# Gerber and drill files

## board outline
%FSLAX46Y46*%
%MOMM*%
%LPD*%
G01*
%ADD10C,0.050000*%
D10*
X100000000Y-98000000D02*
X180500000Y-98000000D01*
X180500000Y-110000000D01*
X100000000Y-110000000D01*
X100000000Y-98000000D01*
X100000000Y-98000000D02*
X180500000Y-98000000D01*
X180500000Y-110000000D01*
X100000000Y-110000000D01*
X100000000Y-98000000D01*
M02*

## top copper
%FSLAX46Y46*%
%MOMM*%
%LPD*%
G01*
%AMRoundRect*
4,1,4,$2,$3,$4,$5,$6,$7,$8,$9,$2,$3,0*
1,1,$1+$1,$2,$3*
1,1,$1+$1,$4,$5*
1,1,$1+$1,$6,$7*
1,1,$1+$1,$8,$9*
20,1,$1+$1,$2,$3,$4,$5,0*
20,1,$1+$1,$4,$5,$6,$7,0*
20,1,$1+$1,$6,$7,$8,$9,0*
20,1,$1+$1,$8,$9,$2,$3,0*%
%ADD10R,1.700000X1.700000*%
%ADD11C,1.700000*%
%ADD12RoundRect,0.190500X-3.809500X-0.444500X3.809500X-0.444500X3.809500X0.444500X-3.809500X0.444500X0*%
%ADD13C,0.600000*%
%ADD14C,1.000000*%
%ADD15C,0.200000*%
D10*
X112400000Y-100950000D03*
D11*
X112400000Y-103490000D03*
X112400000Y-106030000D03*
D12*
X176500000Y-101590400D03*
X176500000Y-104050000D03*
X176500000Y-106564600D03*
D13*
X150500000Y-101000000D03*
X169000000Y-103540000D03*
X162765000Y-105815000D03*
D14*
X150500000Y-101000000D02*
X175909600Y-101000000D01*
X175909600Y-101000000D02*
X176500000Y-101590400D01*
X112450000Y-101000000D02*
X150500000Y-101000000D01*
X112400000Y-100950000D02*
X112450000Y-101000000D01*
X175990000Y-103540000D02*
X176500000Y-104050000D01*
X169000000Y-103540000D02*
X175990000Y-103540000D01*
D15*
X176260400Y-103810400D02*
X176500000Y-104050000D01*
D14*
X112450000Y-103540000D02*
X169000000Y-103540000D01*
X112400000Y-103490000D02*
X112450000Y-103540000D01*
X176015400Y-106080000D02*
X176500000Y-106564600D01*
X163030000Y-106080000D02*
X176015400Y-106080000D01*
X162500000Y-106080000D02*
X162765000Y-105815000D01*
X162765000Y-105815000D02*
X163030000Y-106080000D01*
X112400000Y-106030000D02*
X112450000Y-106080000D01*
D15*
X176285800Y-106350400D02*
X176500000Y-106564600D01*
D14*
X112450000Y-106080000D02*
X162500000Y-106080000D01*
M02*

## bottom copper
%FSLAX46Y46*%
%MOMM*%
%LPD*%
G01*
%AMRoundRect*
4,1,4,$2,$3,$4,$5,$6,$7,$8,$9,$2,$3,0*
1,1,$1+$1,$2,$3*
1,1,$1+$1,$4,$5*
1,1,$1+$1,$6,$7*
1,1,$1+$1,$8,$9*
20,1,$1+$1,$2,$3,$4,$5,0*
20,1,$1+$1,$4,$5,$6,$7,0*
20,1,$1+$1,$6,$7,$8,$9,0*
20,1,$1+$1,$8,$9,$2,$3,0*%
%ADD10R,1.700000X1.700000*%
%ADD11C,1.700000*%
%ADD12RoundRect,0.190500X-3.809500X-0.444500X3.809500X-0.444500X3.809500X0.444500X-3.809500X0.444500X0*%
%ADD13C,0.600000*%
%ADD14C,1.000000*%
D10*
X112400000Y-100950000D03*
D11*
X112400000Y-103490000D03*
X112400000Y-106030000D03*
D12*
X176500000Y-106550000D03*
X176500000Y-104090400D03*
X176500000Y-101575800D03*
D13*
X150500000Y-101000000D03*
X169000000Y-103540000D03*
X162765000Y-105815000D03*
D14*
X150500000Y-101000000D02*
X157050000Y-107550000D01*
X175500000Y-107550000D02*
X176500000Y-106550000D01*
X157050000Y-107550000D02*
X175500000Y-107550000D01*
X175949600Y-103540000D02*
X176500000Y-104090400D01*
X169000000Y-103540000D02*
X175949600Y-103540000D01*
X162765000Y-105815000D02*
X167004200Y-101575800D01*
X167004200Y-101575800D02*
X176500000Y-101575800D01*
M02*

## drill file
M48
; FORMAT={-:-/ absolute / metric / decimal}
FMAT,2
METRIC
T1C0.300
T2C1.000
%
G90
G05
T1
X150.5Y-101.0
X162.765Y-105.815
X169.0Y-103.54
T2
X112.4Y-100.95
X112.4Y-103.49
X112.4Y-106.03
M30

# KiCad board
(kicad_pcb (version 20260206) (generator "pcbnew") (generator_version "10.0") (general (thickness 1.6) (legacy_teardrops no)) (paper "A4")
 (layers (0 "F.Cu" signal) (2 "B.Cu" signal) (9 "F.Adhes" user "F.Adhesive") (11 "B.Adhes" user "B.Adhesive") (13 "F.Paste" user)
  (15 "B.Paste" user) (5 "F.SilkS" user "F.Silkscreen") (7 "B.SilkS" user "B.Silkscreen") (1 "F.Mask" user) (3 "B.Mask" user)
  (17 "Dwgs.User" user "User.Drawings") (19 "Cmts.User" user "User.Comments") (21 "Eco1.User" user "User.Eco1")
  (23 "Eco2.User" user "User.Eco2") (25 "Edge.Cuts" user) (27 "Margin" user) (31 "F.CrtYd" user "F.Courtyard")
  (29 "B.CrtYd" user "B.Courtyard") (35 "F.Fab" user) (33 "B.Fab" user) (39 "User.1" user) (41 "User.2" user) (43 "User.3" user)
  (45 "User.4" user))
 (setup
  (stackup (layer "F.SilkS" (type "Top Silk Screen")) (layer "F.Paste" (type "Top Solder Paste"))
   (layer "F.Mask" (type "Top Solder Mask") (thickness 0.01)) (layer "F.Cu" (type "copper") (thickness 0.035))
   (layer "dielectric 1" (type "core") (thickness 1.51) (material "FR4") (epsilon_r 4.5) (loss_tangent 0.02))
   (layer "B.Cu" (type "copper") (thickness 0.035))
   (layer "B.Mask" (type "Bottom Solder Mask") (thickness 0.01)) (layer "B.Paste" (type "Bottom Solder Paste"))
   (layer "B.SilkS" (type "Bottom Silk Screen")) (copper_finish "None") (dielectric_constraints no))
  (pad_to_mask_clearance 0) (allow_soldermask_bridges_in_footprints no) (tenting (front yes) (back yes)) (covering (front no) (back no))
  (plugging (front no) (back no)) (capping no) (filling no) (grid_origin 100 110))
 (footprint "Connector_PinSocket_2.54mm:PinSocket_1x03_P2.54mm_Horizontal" (layer "F.Cu") (at 112.4 100.95)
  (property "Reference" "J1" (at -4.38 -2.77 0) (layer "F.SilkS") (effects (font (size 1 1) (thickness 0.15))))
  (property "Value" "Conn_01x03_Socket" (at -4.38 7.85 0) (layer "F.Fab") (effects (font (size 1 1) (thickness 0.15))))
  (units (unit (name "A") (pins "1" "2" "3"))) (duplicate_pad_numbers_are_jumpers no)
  (pad "1" thru_hole rect (at 0 0) (size 1.7 1.7) (drill 1) (layers "*.Cu" "*.Mask") (remove_unused_layers no) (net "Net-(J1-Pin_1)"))
  (pad "2" thru_hole circle (at 0 2.54) (size 1.7 1.7) (drill 1) (layers "*.Cu" "*.Mask") (remove_unused_layers no) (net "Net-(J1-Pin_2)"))
  (pad "3" thru_hole circle (at 0 5.08) (size 1.7 1.7) (drill 1) (layers "*.Cu" "*.Mask") (remove_unused_layers no) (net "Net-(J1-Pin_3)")))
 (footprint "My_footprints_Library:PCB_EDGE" (layer "F.Cu") (at 176.5 97.0904)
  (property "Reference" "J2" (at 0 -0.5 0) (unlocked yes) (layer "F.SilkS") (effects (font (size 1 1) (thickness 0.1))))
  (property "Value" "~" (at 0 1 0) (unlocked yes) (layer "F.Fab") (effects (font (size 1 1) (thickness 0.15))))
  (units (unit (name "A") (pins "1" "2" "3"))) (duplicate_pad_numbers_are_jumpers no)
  (pad "1" smd roundrect (at 0 4.5) (size 8 1.27) (layers "F.Cu" "F.Mask" "F.Paste") (roundrect_rratio 0.15) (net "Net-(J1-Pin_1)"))
  (pad "2" smd roundrect (at 0 6.9596) (size 8 1.27) (layers "F.Cu" "F.Mask" "F.Paste") (roundrect_rratio 0.15) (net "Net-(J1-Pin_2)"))
  (pad "3" smd roundrect (at 0 9.4742) (size 8 1.27) (layers "F.Cu" "F.Mask" "F.Paste") (roundrect_rratio 0.15) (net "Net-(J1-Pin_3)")))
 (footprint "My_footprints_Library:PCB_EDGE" (layer "B.Cu") (at 176.5 111.05)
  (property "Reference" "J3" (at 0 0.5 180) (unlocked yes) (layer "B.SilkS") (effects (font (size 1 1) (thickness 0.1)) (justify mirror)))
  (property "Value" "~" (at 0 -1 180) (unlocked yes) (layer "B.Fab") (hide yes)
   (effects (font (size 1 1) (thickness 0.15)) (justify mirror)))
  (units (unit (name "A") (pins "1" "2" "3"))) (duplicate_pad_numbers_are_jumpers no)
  (pad "1" smd roundrect (at 0 -4.5) (size 8 1.27) (layers "B.Cu" "B.Mask" "B.Paste") (roundrect_rratio 0.15) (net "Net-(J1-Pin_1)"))
  (pad "2" smd roundrect (at 0 -6.9596) (size 8 1.27) (layers "B.Cu" "B.Mask" "B.Paste") (roundrect_rratio 0.15) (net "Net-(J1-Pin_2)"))
  (pad "3" smd roundrect (at 0 -9.4742) (size 8 1.27) (layers "B.Cu" "B.Mask" "B.Paste") (roundrect_rratio 0.15) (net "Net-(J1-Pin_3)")))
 (gr_rect (start 100 98) (end 180.5 110) (stroke (width 0.05) (type default)) (fill no) (layer "Edge.Cuts"))
 (segment (start 150.5 101) (end 175.9096 101) (width 1) (layer "F.Cu") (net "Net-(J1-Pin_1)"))
 (segment (start 175.9096 101) (end 176.5 101.5904) (width 1) (layer "F.Cu") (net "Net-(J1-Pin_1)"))
 (segment (start 112.45 101) (end 150.5 101) (width 1) (layer "F.Cu") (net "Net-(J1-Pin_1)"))
 (segment (start 112.4 100.95) (end 112.45 101) (width 1) (layer "F.Cu") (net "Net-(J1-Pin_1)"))
 (via (at 150.5 101) (size 0.6) (drill 0.3) (layers "F.Cu" "B.Cu") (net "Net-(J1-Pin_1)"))
 (segment (start 150.5 101) (end 157.05 107.55) (width 1) (layer "B.Cu") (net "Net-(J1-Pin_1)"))
 (segment (start 175.5 107.55) (end 176.5 106.55) (width 1) (layer "B.Cu") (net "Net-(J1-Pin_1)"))
 (segment (start 157.05 107.55) (end 175.5 107.55) (width 1) (layer "B.Cu") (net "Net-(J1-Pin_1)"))
 (segment (start 175.99 103.54) (end 176.5 104.05) (width 1) (layer "F.Cu") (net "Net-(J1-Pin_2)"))
 (segment (start 169 103.54) (end 175.99 103.54) (width 1) (layer "F.Cu") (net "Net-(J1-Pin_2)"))
 (segment (start 176.2604 103.8104) (end 176.5 104.05) (width 0.2) (layer "F.Cu") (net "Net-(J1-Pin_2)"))
 (segment (start 112.45 103.54) (end 169 103.54) (width 1) (layer "F.Cu") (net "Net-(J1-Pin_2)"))
 (segment (start 112.4 103.49) (end 112.45 103.54) (width 1) (layer "F.Cu") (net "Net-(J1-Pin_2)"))
 (via (at 169 103.54) (size 0.6) (drill 0.3) (layers "F.Cu" "B.Cu") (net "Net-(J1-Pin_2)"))
 (segment (start 175.9496 103.54) (end 176.5 104.0904) (width 1) (layer "B.Cu") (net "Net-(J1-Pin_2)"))
 (segment (start 169 103.54) (end 175.9496 103.54) (width 1) (layer "B.Cu") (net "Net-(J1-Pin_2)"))
 (segment (start 176.0154 106.08) (end 176.5 106.5646) (width 1) (layer "F.Cu") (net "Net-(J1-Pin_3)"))
 (segment (start 163.03 106.08) (end 176.0154 106.08) (width 1) (layer "F.Cu") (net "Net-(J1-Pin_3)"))
 (segment (start 162.5 106.08) (end 162.765 105.815) (width 1) (layer "F.Cu") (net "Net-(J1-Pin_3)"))
 (segment (start 162.765 105.815) (end 163.03 106.08) (width 1) (layer "F.Cu") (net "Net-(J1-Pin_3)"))
 (segment (start 112.4 106.03) (end 112.45 106.08) (width 1) (layer "F.Cu") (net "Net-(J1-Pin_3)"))
 (segment (start 176.2858 106.3504) (end 176.5 106.5646) (width 0.2) (layer "F.Cu") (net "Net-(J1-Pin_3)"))
 (segment (start 112.45 106.08) (end 162.5 106.08) (width 1) (layer "F.Cu") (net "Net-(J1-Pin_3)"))
 (via (at 162.765 105.815) (size 0.6) (drill 0.3) (layers "F.Cu" "B.Cu") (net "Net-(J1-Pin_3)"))
 (segment (start 162.765 105.815) (end 167.0042 101.5758) (width 1) (layer "B.Cu") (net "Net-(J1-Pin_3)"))
 (segment (start 167.0042 101.5758) (end 176.5 101.5758) (width 1) (layer "B.Cu") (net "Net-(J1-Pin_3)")))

